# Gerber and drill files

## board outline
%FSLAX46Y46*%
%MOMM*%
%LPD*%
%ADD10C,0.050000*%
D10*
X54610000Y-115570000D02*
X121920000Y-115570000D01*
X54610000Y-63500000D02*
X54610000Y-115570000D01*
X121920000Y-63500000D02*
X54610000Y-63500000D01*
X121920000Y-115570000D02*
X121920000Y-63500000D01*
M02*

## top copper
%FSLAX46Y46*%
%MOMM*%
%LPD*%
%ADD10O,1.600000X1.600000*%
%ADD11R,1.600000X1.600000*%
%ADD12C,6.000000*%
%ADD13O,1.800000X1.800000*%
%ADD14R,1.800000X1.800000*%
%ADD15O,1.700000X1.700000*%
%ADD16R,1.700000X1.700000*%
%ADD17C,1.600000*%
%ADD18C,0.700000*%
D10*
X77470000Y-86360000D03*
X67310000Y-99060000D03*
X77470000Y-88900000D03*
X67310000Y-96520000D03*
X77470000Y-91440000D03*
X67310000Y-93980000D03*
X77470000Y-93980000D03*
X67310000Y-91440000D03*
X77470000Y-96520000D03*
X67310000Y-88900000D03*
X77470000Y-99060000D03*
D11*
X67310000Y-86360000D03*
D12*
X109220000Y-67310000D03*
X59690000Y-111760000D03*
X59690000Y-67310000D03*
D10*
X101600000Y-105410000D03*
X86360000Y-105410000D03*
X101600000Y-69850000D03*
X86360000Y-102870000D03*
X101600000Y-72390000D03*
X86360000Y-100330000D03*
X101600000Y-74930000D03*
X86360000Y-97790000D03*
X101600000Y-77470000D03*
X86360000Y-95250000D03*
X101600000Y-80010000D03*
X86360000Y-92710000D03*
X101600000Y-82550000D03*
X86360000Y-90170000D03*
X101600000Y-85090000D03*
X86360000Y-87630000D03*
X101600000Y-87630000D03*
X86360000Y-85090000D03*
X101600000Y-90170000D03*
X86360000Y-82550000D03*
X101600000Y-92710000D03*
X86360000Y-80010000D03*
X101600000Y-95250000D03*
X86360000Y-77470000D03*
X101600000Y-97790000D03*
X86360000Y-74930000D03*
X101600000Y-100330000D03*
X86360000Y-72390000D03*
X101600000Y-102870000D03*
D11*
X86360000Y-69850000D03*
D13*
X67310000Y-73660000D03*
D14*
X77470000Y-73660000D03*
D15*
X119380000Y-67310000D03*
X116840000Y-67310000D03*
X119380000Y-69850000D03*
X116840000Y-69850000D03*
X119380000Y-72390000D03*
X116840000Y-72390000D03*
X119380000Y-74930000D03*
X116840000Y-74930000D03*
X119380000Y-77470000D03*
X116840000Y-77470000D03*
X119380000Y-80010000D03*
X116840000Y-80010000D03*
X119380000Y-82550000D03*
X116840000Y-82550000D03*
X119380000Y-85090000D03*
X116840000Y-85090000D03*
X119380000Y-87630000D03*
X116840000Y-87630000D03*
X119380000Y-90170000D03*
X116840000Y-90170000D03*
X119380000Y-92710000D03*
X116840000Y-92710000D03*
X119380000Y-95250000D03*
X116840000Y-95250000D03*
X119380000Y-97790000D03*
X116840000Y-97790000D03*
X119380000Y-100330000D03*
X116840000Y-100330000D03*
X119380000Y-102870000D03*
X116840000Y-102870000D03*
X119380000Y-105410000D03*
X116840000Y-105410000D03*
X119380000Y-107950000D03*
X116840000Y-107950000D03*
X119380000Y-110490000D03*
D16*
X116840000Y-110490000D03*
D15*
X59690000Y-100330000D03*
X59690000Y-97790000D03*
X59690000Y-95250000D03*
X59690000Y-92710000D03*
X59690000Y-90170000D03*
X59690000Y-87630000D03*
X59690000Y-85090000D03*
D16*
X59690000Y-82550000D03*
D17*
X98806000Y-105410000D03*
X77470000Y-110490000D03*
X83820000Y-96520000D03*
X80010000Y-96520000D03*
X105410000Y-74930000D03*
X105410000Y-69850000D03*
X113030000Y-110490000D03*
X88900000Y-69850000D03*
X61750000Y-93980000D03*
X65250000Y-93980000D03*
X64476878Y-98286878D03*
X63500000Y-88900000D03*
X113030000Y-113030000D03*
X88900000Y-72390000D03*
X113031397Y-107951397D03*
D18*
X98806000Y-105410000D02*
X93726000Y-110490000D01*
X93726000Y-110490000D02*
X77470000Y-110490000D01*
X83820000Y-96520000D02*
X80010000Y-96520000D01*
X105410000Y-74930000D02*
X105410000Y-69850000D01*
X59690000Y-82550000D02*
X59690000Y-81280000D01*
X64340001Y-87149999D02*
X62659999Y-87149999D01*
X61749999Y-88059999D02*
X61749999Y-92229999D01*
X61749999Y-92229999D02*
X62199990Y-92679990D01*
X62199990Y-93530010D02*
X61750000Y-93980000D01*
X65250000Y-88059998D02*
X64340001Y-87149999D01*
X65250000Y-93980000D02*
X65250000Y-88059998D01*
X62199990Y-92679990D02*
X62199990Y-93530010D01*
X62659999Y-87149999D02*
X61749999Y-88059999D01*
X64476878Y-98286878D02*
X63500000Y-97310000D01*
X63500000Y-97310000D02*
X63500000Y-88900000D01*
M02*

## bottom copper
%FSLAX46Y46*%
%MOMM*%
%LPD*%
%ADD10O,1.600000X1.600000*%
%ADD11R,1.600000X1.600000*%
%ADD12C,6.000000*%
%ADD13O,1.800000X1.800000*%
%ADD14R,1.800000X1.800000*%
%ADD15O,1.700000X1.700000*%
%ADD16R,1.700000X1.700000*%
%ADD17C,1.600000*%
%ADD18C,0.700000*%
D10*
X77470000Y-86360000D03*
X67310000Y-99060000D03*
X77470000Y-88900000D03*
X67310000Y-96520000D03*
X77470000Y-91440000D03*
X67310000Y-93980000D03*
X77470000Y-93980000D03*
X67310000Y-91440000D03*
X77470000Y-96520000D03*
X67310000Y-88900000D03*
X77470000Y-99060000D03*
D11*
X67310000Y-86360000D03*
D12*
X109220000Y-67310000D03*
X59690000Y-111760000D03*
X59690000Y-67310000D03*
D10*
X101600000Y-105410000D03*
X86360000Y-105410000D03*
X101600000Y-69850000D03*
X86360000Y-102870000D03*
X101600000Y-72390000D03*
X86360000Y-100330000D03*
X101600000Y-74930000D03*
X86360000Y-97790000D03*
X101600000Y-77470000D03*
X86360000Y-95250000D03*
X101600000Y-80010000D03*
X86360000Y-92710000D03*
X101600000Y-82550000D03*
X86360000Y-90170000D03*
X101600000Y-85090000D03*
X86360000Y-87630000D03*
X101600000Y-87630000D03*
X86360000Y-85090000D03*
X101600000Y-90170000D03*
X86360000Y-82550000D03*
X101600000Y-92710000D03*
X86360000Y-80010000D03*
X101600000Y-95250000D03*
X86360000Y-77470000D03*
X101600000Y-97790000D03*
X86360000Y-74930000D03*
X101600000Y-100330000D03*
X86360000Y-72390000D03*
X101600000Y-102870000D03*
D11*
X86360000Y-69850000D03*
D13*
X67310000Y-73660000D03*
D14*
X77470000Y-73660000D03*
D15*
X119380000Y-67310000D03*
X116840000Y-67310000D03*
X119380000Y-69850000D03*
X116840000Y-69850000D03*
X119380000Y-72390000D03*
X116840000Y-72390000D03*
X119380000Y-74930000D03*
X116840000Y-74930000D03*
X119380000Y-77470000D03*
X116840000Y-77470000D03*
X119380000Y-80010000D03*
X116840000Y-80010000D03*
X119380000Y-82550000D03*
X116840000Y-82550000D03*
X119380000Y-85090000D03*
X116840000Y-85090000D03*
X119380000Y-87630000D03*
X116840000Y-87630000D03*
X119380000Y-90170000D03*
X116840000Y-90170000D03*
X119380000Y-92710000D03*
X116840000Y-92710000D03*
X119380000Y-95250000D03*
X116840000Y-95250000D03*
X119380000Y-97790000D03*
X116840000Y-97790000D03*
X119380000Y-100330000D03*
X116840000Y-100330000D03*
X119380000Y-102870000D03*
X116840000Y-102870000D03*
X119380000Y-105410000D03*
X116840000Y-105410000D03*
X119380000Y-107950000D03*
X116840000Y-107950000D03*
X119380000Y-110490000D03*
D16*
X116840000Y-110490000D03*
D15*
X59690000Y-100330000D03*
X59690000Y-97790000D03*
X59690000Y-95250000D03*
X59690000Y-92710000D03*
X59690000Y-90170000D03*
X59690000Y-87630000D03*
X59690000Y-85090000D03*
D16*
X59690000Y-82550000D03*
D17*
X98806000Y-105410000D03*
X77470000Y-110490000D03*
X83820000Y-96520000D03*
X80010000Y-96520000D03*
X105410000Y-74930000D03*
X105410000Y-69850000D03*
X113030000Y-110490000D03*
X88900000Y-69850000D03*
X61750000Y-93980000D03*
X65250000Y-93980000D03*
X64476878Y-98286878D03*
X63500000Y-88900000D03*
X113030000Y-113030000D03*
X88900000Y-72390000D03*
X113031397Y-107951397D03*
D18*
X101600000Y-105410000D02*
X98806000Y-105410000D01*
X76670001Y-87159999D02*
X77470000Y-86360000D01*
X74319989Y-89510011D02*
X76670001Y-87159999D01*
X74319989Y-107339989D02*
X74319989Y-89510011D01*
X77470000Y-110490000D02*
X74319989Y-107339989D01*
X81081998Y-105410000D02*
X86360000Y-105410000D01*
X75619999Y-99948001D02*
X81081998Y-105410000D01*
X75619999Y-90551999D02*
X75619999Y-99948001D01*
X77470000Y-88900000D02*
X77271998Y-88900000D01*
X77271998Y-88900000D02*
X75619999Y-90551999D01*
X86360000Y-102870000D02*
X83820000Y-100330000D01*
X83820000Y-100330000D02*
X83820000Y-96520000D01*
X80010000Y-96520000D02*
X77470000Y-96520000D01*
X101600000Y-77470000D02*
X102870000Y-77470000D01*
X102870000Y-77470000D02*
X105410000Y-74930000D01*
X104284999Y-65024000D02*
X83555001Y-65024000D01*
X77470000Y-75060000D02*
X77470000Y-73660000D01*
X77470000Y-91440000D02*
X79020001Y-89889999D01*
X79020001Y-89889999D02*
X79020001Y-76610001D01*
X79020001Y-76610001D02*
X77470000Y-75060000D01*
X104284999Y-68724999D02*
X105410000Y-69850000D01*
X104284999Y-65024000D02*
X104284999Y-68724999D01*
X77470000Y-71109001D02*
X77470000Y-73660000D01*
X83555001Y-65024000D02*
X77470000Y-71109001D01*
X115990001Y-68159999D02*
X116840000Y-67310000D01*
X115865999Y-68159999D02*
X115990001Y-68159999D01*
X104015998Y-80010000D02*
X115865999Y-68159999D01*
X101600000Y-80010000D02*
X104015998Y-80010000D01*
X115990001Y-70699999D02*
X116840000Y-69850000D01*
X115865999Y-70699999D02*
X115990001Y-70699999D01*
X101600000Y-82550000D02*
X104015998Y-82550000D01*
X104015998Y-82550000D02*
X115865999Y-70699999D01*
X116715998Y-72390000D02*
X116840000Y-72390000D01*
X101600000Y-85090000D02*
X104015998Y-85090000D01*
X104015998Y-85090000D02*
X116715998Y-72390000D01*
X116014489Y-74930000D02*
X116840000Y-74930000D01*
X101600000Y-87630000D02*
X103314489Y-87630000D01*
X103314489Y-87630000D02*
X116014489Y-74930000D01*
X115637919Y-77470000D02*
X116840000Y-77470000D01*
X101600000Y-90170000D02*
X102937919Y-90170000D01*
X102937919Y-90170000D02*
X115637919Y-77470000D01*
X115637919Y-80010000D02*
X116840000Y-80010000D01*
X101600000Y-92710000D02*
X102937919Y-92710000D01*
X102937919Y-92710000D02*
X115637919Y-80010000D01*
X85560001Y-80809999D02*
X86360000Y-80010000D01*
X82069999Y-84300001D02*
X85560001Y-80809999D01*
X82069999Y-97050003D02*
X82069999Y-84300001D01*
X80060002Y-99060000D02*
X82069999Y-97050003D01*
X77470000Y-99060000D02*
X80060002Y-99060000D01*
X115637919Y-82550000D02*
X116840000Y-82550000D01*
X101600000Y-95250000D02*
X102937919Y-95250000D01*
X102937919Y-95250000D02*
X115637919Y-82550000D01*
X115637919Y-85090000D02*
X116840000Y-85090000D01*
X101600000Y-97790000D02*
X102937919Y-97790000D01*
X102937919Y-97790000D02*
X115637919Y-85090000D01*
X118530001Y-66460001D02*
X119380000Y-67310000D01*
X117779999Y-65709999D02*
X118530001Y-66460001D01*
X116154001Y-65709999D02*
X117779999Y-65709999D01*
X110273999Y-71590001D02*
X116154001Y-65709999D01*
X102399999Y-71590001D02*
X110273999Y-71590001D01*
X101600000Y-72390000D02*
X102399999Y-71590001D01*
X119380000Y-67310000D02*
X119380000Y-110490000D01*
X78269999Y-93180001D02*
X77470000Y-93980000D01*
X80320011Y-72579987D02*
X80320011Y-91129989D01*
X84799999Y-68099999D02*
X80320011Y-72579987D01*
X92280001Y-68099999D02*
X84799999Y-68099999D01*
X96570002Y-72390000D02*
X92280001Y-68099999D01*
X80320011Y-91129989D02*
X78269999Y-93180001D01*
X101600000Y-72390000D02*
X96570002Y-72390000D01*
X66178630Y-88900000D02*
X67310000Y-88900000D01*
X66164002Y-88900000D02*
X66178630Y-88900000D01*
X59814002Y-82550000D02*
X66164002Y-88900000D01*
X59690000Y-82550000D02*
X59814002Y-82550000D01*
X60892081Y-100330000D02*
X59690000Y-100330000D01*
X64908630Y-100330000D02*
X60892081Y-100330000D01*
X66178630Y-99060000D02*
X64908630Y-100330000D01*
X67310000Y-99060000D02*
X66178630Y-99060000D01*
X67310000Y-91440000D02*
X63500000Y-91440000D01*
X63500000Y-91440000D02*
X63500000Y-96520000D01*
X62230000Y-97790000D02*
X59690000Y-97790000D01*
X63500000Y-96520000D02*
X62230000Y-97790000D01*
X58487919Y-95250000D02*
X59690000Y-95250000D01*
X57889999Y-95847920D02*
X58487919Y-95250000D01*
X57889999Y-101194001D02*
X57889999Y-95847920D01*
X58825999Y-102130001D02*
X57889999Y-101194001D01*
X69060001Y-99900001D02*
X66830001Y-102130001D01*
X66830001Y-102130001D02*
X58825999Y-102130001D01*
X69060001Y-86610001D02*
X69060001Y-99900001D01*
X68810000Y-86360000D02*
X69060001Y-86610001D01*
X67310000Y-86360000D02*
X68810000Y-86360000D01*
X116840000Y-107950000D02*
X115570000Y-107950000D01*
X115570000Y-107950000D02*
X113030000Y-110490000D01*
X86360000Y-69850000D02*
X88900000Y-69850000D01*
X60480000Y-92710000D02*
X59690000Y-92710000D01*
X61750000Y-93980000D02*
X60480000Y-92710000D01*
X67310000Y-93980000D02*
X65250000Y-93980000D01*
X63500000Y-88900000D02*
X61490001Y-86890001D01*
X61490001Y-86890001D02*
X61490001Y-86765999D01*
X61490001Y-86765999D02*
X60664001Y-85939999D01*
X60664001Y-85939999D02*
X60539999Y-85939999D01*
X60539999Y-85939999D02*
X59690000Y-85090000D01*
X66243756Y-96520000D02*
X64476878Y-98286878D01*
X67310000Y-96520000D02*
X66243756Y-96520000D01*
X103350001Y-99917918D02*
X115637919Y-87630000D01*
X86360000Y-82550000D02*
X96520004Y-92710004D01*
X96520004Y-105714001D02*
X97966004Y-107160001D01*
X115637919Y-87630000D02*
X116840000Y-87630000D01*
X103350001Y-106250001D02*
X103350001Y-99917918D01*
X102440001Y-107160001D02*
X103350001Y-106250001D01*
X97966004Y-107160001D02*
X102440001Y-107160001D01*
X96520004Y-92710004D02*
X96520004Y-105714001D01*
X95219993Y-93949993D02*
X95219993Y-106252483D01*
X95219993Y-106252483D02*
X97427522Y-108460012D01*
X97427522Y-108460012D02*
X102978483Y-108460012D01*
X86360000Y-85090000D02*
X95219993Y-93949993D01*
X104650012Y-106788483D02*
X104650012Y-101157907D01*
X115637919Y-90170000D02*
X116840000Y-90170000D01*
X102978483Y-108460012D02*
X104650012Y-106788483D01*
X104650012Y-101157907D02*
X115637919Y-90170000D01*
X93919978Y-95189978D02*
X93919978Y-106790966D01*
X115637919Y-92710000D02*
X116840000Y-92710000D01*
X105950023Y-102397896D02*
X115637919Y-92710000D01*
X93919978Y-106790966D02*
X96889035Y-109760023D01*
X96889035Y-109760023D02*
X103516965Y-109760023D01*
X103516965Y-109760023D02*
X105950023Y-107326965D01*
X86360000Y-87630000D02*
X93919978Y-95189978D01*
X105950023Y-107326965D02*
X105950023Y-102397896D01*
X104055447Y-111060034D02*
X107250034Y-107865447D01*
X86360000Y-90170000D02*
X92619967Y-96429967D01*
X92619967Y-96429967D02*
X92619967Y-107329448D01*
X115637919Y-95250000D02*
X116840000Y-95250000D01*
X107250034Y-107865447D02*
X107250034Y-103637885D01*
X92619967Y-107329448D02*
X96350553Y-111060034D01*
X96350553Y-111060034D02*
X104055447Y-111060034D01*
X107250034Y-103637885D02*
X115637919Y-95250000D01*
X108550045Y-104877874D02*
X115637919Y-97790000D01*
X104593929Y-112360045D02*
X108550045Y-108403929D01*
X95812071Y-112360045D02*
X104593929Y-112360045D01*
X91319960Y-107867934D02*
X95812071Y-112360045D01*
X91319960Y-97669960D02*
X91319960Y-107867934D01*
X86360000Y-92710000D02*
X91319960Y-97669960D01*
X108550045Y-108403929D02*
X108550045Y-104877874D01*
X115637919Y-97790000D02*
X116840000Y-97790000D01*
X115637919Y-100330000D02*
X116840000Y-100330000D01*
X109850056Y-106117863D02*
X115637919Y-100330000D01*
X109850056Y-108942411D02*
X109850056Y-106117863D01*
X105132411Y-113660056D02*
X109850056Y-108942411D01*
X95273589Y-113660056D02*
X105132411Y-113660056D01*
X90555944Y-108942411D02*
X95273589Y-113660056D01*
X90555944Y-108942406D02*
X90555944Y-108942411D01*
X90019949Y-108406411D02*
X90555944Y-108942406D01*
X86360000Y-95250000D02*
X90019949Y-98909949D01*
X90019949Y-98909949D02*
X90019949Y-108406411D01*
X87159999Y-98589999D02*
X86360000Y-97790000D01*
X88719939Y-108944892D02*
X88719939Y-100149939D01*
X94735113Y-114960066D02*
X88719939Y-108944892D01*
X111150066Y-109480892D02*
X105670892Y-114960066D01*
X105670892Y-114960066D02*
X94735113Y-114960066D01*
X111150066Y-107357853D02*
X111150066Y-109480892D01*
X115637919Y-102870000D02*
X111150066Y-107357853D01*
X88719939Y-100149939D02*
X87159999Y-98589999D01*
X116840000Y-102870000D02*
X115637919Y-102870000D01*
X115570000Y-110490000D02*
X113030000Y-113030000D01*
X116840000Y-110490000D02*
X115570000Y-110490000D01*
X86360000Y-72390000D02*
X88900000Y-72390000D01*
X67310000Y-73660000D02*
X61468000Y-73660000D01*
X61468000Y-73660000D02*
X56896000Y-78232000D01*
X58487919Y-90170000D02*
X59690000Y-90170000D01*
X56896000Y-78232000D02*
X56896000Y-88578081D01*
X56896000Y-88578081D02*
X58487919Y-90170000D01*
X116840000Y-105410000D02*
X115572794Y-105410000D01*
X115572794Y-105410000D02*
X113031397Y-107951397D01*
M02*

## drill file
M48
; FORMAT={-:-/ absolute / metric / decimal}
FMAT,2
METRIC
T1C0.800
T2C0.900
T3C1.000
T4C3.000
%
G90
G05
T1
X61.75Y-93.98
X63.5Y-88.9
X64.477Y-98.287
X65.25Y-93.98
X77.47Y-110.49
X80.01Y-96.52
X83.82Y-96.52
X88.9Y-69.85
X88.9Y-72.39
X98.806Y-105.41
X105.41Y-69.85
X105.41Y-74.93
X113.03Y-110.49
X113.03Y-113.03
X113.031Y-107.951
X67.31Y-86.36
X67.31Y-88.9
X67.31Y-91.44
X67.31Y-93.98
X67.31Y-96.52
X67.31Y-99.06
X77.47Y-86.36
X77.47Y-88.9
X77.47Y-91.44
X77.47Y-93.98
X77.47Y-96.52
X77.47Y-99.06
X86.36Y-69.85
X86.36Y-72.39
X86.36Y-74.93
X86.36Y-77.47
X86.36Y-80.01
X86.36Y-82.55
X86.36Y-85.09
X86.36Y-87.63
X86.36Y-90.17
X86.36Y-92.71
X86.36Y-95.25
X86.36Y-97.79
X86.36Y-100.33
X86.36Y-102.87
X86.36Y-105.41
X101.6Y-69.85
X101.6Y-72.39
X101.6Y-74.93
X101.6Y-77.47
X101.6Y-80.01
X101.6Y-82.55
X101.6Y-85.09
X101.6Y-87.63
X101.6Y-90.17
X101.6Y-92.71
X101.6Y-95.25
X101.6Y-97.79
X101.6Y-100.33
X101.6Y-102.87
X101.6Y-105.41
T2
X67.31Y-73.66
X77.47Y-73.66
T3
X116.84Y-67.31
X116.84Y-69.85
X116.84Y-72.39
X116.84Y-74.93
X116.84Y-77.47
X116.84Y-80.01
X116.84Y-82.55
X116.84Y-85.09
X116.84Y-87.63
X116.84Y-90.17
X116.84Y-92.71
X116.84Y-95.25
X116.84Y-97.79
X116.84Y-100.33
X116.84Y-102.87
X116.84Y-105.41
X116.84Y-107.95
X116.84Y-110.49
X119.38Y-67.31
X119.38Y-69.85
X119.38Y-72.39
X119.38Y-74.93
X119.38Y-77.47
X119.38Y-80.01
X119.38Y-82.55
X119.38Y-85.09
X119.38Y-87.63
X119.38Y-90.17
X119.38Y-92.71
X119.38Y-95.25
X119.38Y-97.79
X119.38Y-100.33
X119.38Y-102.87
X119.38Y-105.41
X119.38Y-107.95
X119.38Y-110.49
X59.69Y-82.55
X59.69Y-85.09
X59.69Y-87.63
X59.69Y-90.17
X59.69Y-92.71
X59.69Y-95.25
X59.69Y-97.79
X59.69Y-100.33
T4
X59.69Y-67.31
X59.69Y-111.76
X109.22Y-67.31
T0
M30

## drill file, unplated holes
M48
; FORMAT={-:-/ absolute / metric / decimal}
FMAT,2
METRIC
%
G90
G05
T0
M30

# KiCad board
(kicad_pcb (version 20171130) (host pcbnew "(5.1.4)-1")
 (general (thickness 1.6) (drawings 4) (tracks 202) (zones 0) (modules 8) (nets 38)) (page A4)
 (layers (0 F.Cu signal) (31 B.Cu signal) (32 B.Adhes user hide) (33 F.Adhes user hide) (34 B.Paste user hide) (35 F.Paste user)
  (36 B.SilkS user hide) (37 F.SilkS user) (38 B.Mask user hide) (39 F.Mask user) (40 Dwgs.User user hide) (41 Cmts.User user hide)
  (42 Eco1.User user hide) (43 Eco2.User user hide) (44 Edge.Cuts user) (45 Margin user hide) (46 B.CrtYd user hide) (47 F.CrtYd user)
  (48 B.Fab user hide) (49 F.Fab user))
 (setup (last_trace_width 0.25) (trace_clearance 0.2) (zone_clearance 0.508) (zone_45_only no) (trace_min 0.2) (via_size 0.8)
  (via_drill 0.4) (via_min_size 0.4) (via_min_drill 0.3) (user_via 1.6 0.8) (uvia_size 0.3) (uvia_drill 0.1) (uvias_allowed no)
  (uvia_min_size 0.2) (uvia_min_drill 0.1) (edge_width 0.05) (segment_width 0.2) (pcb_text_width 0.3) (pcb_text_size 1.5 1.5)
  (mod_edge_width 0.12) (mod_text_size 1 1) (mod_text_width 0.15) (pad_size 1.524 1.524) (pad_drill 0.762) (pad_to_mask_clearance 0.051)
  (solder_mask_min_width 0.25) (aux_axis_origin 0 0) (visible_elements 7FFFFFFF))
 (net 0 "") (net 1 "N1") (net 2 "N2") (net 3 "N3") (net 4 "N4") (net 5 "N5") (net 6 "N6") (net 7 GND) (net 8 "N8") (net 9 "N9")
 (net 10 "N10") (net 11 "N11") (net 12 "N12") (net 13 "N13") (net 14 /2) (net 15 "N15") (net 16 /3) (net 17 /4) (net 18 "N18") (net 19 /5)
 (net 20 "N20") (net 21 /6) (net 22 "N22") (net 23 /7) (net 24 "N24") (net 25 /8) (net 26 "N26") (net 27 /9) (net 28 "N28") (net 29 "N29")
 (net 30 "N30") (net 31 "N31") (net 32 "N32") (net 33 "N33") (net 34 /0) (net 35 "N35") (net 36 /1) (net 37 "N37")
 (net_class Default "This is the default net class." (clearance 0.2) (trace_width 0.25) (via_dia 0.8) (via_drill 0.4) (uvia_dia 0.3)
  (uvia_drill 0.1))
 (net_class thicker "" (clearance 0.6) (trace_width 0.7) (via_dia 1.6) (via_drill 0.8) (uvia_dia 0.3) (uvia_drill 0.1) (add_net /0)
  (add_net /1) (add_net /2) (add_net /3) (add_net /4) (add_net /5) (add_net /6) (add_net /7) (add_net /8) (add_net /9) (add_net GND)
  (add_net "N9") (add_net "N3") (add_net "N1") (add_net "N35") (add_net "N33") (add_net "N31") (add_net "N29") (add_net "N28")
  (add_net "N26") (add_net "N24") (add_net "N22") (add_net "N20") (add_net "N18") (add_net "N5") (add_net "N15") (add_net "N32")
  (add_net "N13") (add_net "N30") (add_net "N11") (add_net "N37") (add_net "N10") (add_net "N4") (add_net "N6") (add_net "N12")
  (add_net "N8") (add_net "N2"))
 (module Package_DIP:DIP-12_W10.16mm (layer F.Cu) (at 67.31 86.36)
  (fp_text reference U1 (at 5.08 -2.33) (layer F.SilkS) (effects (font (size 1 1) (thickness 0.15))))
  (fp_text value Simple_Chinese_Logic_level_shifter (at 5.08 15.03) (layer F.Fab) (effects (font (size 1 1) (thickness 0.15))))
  (pad 10 thru_hole oval (at 10.16 0) (size 1.6 1.6) (drill 0.8) (layers *.Cu *.Mask) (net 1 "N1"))
  (pad 5 thru_hole oval (at 0 12.7) (size 1.6 1.6) (drill 0.8) (layers *.Cu *.Mask) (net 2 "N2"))
  (pad 9 thru_hole oval (at 10.16 2.54) (size 1.6 1.6) (drill 0.8) (layers *.Cu *.Mask) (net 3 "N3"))
  (pad 4 thru_hole oval (at 0 10.16) (size 1.6 1.6) (drill 0.8) (layers *.Cu *.Mask) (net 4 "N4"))
  (pad 11 thru_hole oval (at 10.16 5.08) (size 1.6 1.6) (drill 0.8) (layers *.Cu *.Mask) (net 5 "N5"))
  (pad 12 thru_hole oval (at 0 7.62) (size 1.6 1.6) (drill 0.8) (layers *.Cu *.Mask) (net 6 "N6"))
  (pad 6 thru_hole oval (at 10.16 7.62) (size 1.6 1.6) (drill 0.8) (layers *.Cu *.Mask) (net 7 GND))
  (pad 1 thru_hole oval (at 0 5.08) (size 1.6 1.6) (drill 0.8) (layers *.Cu *.Mask) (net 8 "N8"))
  (pad 8 thru_hole oval (at 10.16 10.16) (size 1.6 1.6) (drill 0.8) (layers *.Cu *.Mask) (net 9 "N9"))
  (pad 3 thru_hole oval (at 0 2.54) (size 1.6 1.6) (drill 0.8) (layers *.Cu *.Mask) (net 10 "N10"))
  (pad 7 thru_hole oval (at 10.16 12.7) (size 1.6 1.6) (drill 0.8) (layers *.Cu *.Mask) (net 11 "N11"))
  (pad 2 thru_hole rect (at 0 0) (size 1.6 1.6) (drill 0.8) (layers *.Cu *.Mask) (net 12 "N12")))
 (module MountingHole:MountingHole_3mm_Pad (layer F.Cu) (at 109.22 67.31)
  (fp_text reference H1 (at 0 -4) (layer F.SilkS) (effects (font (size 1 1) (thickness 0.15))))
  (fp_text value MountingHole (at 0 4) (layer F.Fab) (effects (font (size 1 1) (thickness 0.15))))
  (pad 1 thru_hole circle (at 0 0) (size 6 6) (drill 3) (layers *.Cu *.Mask)))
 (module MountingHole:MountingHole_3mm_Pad (layer F.Cu) (at 59.69 111.76)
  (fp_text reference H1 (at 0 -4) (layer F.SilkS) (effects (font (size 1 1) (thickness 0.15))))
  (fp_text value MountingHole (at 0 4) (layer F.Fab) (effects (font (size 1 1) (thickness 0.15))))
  (pad 1 thru_hole circle (at 0 0) (size 6 6) (drill 3) (layers *.Cu *.Mask)))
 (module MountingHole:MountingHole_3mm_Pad (layer F.Cu) (at 59.69 67.31)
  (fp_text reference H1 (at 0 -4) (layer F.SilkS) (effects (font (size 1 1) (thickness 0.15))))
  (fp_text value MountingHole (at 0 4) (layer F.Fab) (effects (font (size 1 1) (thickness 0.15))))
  (pad 1 thru_hole circle (at 0 0) (size 6 6) (drill 3) (layers *.Cu *.Mask)))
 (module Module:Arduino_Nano (layer F.Cu) (at 86.36 69.85)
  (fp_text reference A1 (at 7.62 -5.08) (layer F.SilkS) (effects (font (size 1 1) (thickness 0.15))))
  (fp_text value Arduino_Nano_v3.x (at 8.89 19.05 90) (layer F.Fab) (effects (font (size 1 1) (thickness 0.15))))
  (pad 16 thru_hole oval (at 15.24 35.56) (size 1.6 1.6) (drill 0.8) (layers *.Cu *.Mask) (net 1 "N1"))
  (pad 15 thru_hole oval (at 0 35.56) (size 1.6 1.6) (drill 0.8) (layers *.Cu *.Mask) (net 3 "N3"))
  (pad 30 thru_hole oval (at 15.24 0) (size 1.6 1.6) (drill 0.8) (layers *.Cu *.Mask) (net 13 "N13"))
  (pad 14 thru_hole oval (at 0 33.02) (size 1.6 1.6) (drill 0.8) (layers *.Cu *.Mask) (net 9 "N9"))
  (pad 29 thru_hole oval (at 15.24 2.54) (size 1.6 1.6) (drill 0.8) (layers *.Cu *.Mask) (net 7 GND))
  (pad 13 thru_hole oval (at 0 30.48) (size 1.6 1.6) (drill 0.8) (layers *.Cu *.Mask) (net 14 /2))
  (pad 28 thru_hole oval (at 15.24 5.08) (size 1.6 1.6) (drill 0.8) (layers *.Cu *.Mask) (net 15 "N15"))
  (pad 12 thru_hole oval (at 0 27.94) (size 1.6 1.6) (drill 0.8) (layers *.Cu *.Mask) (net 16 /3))
  (pad 27 thru_hole oval (at 15.24 7.62) (size 1.6 1.6) (drill 0.8) (layers *.Cu *.Mask) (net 5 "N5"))
  (pad 11 thru_hole oval (at 0 25.4) (size 1.6 1.6) (drill 0.8) (layers *.Cu *.Mask) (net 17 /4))
  (pad 26 thru_hole oval (at 15.24 10.16) (size 1.6 1.6) (drill 0.8) (layers *.Cu *.Mask) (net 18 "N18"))
  (pad 10 thru_hole oval (at 0 22.86) (size 1.6 1.6) (drill 0.8) (layers *.Cu *.Mask) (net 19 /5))
  (pad 25 thru_hole oval (at 15.24 12.7) (size 1.6 1.6) (drill 0.8) (layers *.Cu *.Mask) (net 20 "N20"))
  (pad 9 thru_hole oval (at 0 20.32) (size 1.6 1.6) (drill 0.8) (layers *.Cu *.Mask) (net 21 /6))
  (pad 24 thru_hole oval (at 15.24 15.24) (size 1.6 1.6) (drill 0.8) (layers *.Cu *.Mask) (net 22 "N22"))
  (pad 8 thru_hole oval (at 0 17.78) (size 1.6 1.6) (drill 0.8) (layers *.Cu *.Mask) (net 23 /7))
  (pad 23 thru_hole oval (at 15.24 17.78) (size 1.6 1.6) (drill 0.8) (layers *.Cu *.Mask) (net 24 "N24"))
  (pad 7 thru_hole oval (at 0 15.24) (size 1.6 1.6) (drill 0.8) (layers *.Cu *.Mask) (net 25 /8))
  (pad 22 thru_hole oval (at 15.24 20.32) (size 1.6 1.6) (drill 0.8) (layers *.Cu *.Mask) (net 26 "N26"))
  (pad 6 thru_hole oval (at 0 12.7) (size 1.6 1.6) (drill 0.8) (layers *.Cu *.Mask) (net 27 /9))
  (pad 21 thru_hole oval (at 15.24 22.86) (size 1.6 1.6) (drill 0.8) (layers *.Cu *.Mask) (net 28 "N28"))
  (pad 5 thru_hole oval (at 0 10.16) (size 1.6 1.6) (drill 0.8) (layers *.Cu *.Mask) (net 11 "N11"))
  (pad 20 thru_hole oval (at 15.24 25.4) (size 1.6 1.6) (drill 0.8) (layers *.Cu *.Mask) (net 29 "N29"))
  (pad 4 thru_hole oval (at 0 7.62) (size 1.6 1.6) (drill 0.8) (layers *.Cu *.Mask) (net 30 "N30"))
  (pad 19 thru_hole oval (at 15.24 27.94) (size 1.6 1.6) (drill 0.8) (layers *.Cu *.Mask) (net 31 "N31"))
  (pad 3 thru_hole oval (at 0 5.08) (size 1.6 1.6) (drill 0.8) (layers *.Cu *.Mask) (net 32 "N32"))
  (pad 18 thru_hole oval (at 15.24 30.48) (size 1.6 1.6) (drill 0.8) (layers *.Cu *.Mask) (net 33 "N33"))
  (pad 2 thru_hole oval (at 0 2.54) (size 1.6 1.6) (drill 0.8) (layers *.Cu *.Mask) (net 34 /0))
  (pad 17 thru_hole oval (at 15.24 33.02) (size 1.6 1.6) (drill 0.8) (layers *.Cu *.Mask) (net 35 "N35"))
  (pad 1 thru_hole rect (at 0 0) (size 1.6 1.6) (drill 0.8) (layers *.Cu *.Mask) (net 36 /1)))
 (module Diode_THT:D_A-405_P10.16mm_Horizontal (layer F.Cu) (at 77.47 73.66 180)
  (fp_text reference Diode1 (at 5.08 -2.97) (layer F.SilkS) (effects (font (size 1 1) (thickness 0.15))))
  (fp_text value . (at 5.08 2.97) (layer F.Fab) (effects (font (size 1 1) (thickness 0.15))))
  (pad 2 thru_hole oval (at 10.16 0 180) (size 1.8 1.8) (drill 0.9) (layers *.Cu *.Mask) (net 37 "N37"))
  (pad 1 thru_hole rect (at 0 0 180) (size 1.8 1.8) (drill 0.9) (layers *.Cu *.Mask) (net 5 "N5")))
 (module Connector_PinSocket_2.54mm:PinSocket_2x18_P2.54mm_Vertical (layer F.Cu) (at 116.84 110.49 180)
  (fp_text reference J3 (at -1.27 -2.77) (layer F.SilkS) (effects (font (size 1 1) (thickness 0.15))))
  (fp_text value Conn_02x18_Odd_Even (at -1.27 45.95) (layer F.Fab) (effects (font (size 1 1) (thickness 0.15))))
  (pad 36 thru_hole oval (at -2.54 43.18 180) (size 1.7 1.7) (drill 1) (layers *.Cu *.Mask) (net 7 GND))
  (pad 35 thru_hole oval (at 0 43.18 180) (size 1.7 1.7) (drill 1) (layers *.Cu *.Mask) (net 18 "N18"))
  (pad 34 thru_hole oval (at -2.54 40.64 180) (size 1.7 1.7) (drill 1) (layers *.Cu *.Mask) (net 7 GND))
  (pad 33 thru_hole oval (at 0 40.64 180) (size 1.7 1.7) (drill 1) (layers *.Cu *.Mask) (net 20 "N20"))
  (pad 32 thru_hole oval (at -2.54 38.1 180) (size 1.7 1.7) (drill 1) (layers *.Cu *.Mask) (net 7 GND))
  (pad 31 thru_hole oval (at 0 38.1 180) (size 1.7 1.7) (drill 1) (layers *.Cu *.Mask) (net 22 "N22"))
  (pad 30 thru_hole oval (at -2.54 35.56 180) (size 1.7 1.7) (drill 1) (layers *.Cu *.Mask) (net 7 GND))
  (pad 29 thru_hole oval (at 0 35.56 180) (size 1.7 1.7) (drill 1) (layers *.Cu *.Mask) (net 24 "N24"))
  (pad 28 thru_hole oval (at -2.54 33.02 180) (size 1.7 1.7) (drill 1) (layers *.Cu *.Mask) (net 7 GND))
  (pad 27 thru_hole oval (at 0 33.02 180) (size 1.7 1.7) (drill 1) (layers *.Cu *.Mask) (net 26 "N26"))
  (pad 26 thru_hole oval (at -2.54 30.48 180) (size 1.7 1.7) (drill 1) (layers *.Cu *.Mask) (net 7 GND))
  (pad 25 thru_hole oval (at 0 30.48 180) (size 1.7 1.7) (drill 1) (layers *.Cu *.Mask) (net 28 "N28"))
  (pad 24 thru_hole oval (at -2.54 27.94 180) (size 1.7 1.7) (drill 1) (layers *.Cu *.Mask) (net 7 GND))
  (pad 23 thru_hole oval (at 0 27.94 180) (size 1.7 1.7) (drill 1) (layers *.Cu *.Mask) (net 29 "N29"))
  (pad 22 thru_hole oval (at -2.54 25.4 180) (size 1.7 1.7) (drill 1) (layers *.Cu *.Mask) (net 7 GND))
  (pad 21 thru_hole oval (at 0 25.4 180) (size 1.7 1.7) (drill 1) (layers *.Cu *.Mask) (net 31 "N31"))
  (pad 20 thru_hole oval (at -2.54 22.86 180) (size 1.7 1.7) (drill 1) (layers *.Cu *.Mask) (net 7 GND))
  (pad 19 thru_hole oval (at 0 22.86 180) (size 1.7 1.7) (drill 1) (layers *.Cu *.Mask) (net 27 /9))
  (pad 18 thru_hole oval (at -2.54 20.32 180) (size 1.7 1.7) (drill 1) (layers *.Cu *.Mask) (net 7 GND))
  (pad 17 thru_hole oval (at 0 20.32 180) (size 1.7 1.7) (drill 1) (layers *.Cu *.Mask) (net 25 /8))
  (pad 16 thru_hole oval (at -2.54 17.78 180) (size 1.7 1.7) (drill 1) (layers *.Cu *.Mask) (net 7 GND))
  (pad 15 thru_hole oval (at 0 17.78 180) (size 1.7 1.7) (drill 1) (layers *.Cu *.Mask) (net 23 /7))
  (pad 14 thru_hole oval (at -2.54 15.24 180) (size 1.7 1.7) (drill 1) (layers *.Cu *.Mask) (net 7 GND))
  (pad 13 thru_hole oval (at 0 15.24 180) (size 1.7 1.7) (drill 1) (layers *.Cu *.Mask) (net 21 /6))
  (pad 12 thru_hole oval (at -2.54 12.7 180) (size 1.7 1.7) (drill 1) (layers *.Cu *.Mask) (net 7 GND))
  (pad 11 thru_hole oval (at 0 12.7 180) (size 1.7 1.7) (drill 1) (layers *.Cu *.Mask) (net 19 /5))
  (pad 10 thru_hole oval (at -2.54 10.16 180) (size 1.7 1.7) (drill 1) (layers *.Cu *.Mask) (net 7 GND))
  (pad 9 thru_hole oval (at 0 10.16 180) (size 1.7 1.7) (drill 1) (layers *.Cu *.Mask) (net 17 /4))
  (pad 8 thru_hole oval (at -2.54 7.62 180) (size 1.7 1.7) (drill 1) (layers *.Cu *.Mask) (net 7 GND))
  (pad 7 thru_hole oval (at 0 7.62 180) (size 1.7 1.7) (drill 1) (layers *.Cu *.Mask) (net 16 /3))
  (pad 6 thru_hole oval (at -2.54 5.08 180) (size 1.7 1.7) (drill 1) (layers *.Cu *.Mask) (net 7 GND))
  (pad 5 thru_hole oval (at 0 5.08 180) (size 1.7 1.7) (drill 1) (layers *.Cu *.Mask) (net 14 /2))
  (pad 4 thru_hole oval (at -2.54 2.54 180) (size 1.7 1.7) (drill 1) (layers *.Cu *.Mask) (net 7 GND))
  (pad 3 thru_hole oval (at 0 2.54 180) (size 1.7 1.7) (drill 1) (layers *.Cu *.Mask) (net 36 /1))
  (pad 2 thru_hole oval (at -2.54 0 180) (size 1.7 1.7) (drill 1) (layers *.Cu *.Mask) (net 7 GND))
  (pad 1 thru_hole rect (at 0 0 180) (size 1.7 1.7) (drill 1) (layers *.Cu *.Mask) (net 34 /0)))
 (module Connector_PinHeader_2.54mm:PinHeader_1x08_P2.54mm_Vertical (layer F.Cu) (at 59.69 82.55)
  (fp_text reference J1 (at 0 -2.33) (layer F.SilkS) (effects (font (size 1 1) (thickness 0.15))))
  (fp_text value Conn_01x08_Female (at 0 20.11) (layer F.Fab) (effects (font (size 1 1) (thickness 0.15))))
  (pad 8 thru_hole oval (at 0 17.78) (size 1.7 1.7) (drill 1) (layers *.Cu *.Mask) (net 2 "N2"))
  (pad 7 thru_hole oval (at 0 15.24) (size 1.7 1.7) (drill 1) (layers *.Cu *.Mask) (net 8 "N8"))
  (pad 6 thru_hole oval (at 0 12.7) (size 1.7 1.7) (drill 1) (layers *.Cu *.Mask) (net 12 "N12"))
  (pad 5 thru_hole oval (at 0 10.16) (size 1.7 1.7) (drill 1) (layers *.Cu *.Mask) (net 6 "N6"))
  (pad 4 thru_hole oval (at 0 7.62) (size 1.7 1.7) (drill 1) (layers *.Cu *.Mask) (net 37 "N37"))
  (pad 3 thru_hole oval (at 0 5.08) (size 1.7 1.7) (drill 1) (layers *.Cu *.Mask) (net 6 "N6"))
  (pad 2 thru_hole oval (at 0 2.54) (size 1.7 1.7) (drill 1) (layers *.Cu *.Mask) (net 4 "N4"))
  (pad 1 thru_hole rect (at 0 0) (size 1.7 1.7) (drill 1) (layers *.Cu *.Mask) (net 10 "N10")))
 (gr_line (start 54.61 115.57) (end 121.92 115.57) (layer Edge.Cuts) (width 0.05))
 (gr_line (start 54.61 63.5) (end 54.61 115.57) (layer Edge.Cuts) (width 0.05))
 (gr_line (start 121.92 63.5) (end 54.61 63.5) (layer Edge.Cuts) (width 0.05))
 (gr_line (start 121.92 115.57) (end 121.92 63.5) (layer Edge.Cuts) (width 0.05))
 (via (at 98.806 105.41) (size 1.6) (drill 0.8) (layers F.Cu B.Cu) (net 1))
 (segment (start 101.6 105.41) (end 98.806 105.41) (width 0.7) (layer B.Cu) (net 1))
 (via (at 77.47 110.49) (size 1.6) (drill 0.8) (layers F.Cu B.Cu) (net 1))
 (segment (start 76.670001 87.159999) (end 77.47 86.36) (width 0.7) (layer B.Cu) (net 1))
 (segment (start 74.319989 89.510011) (end 76.670001 87.159999) (width 0.7) (layer B.Cu) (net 1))
 (segment (start 74.319989 107.339989) (end 74.319989 89.510011) (width 0.7) (layer B.Cu) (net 1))
 (segment (start 77.47 110.49) (end 74.319989 107.339989) (width 0.7) (layer B.Cu) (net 1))
 (segment (start 98.806 105.41) (end 93.726 110.49) (width 0.7) (layer F.Cu) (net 1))
 (segment (start 93.726 110.49) (end 77.47 110.49) (width 0.7) (layer F.Cu) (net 1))
 (segment (start 81.081998 105.41) (end 86.36 105.41) (width 0.7) (layer B.Cu) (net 3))
 (segment (start 75.619999 99.948001) (end 81.081998 105.41) (width 0.7) (layer B.Cu) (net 3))
 (segment (start 75.619999 90.551999) (end 75.619999 99.948001) (width 0.7) (layer B.Cu) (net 3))
 (segment (start 77.47 88.9) (end 77.271998 88.9) (width 0.7) (layer B.Cu) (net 3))
 (segment (start 77.271998 88.9) (end 75.619999 90.551999) (width 0.7) (layer B.Cu) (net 3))
 (segment (start 86.36 102.87) (end 83.82 100.33) (width 0.7) (layer B.Cu) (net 9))
 (via (at 83.82 96.52) (size 1.6) (drill 0.8) (layers F.Cu B.Cu) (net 9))
 (segment (start 83.82 100.33) (end 83.82 96.52) (width 0.7) (layer B.Cu) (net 9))
 (via (at 80.01 96.52) (size 1.6) (drill 0.8) (layers F.Cu B.Cu) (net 9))
 (segment (start 83.82 96.52) (end 80.01 96.52) (width 0.7) (layer F.Cu) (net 9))
 (segment (start 80.01 96.52) (end 77.47 96.52) (width 0.7) (layer B.Cu) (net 9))
 (via (at 105.41 74.93) (size 1.6) (drill 0.8) (layers F.Cu B.Cu) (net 5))
 (segment (start 101.6 77.47) (end 102.87 77.47) (width 0.7) (layer B.Cu) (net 5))
 (segment (start 102.87 77.47) (end 105.41 74.93) (width 0.7) (layer B.Cu) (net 5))
 (via (at 105.41 69.85) (size 1.6) (drill 0.8) (layers F.Cu B.Cu) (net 5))
 (segment (start 105.41 74.93) (end 105.41 69.85) (width 0.7) (layer F.Cu) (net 5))
 (segment (start 104.284999 65.024) (end 83.555001 65.024) (width 0.7) (layer B.Cu) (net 5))
 (segment (start 77.47 75.06) (end 77.47 73.66) (width 0.7) (layer B.Cu) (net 5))
 (segment (start 77.47 91.44) (end 79.020001 89.889999) (width 0.7) (layer B.Cu) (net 5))
 (segment (start 79.020001 89.889999) (end 79.020001 76.610001) (width 0.7) (layer B.Cu) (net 5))
 (segment (start 79.020001 76.610001) (end 77.47 75.06) (width 0.7) (layer B.Cu) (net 5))
 (segment (start 104.284999 68.724999) (end 105.41 69.85) (width 0.7) (layer B.Cu) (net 5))
 (segment (start 104.284999 65.024) (end 104.284999 68.724999) (width 0.7) (layer B.Cu) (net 5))
 (segment (start 77.47 71.109001) (end 77.47 73.66) (width 0.7) (layer B.Cu) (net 5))
 (segment (start 83.555001 65.024) (end 77.47 71.109001) (width 0.7) (layer B.Cu) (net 5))
 (segment (start 115.990001 68.159999) (end 116.84 67.31) (width 0.7) (layer B.Cu) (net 18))
 (segment (start 115.865999 68.159999) (end 115.990001 68.159999) (width 0.7) (layer B.Cu) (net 18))
 (segment (start 104.015998 80.01) (end 115.865999 68.159999) (width 0.7) (layer B.Cu) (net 18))
 (segment (start 101.6 80.01) (end 104.015998 80.01) (width 0.7) (layer B.Cu) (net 18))
 (segment (start 115.990001 70.699999) (end 116.84 69.85) (width 0.7) (layer B.Cu) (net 20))
 (segment (start 115.865999 70.699999) (end 115.990001 70.699999) (width 0.7) (layer B.Cu) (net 20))
 (segment (start 101.6 82.55) (end 104.015998 82.55) (width 0.7) (layer B.Cu) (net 20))
 (segment (start 104.015998 82.55) (end 115.865999 70.699999) (width 0.7) (layer B.Cu) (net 20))
 (segment (start 116.715998 72.39) (end 116.84 72.39) (width 0.7) (layer B.Cu) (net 22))
 (segment (start 101.6 85.09) (end 104.015998 85.09) (width 0.7) (layer B.Cu) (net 22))
 (segment (start 104.015998 85.09) (end 116.715998 72.39) (width 0.7) (layer B.Cu) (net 22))
 (segment (start 116.014489 74.93) (end 116.84 74.93) (width 0.7) (layer B.Cu) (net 24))
 (segment (start 101.6 87.63) (end 103.314489 87.63) (width 0.7) (layer B.Cu) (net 24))
 (segment (start 103.314489 87.63) (end 116.014489 74.93) (width 0.7) (layer B.Cu) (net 24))
 (segment (start 115.637919 77.47) (end 116.84 77.47) (width 0.7) (layer B.Cu) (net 26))
 (segment (start 101.6 90.17) (end 102.937919 90.17) (width 0.7) (layer B.Cu) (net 26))
 (segment (start 102.937919 90.17) (end 115.637919 77.47) (width 0.7) (layer B.Cu) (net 26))
 (segment (start 115.637919 80.01) (end 116.84 80.01) (width 0.7) (layer B.Cu) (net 28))
 (segment (start 101.6 92.71) (end 102.937919 92.71) (width 0.7) (layer B.Cu) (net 28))
 (segment (start 102.937919 92.71) (end 115.637919 80.01) (width 0.7) (layer B.Cu) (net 28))
 (segment (start 85.560001 80.809999) (end 86.36 80.01) (width 0.7) (layer B.Cu) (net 11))
 (segment (start 82.069999 84.300001) (end 85.560001 80.809999) (width 0.7) (layer B.Cu) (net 11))
 (segment (start 82.069999 97.050003) (end 82.069999 84.300001) (width 0.7) (layer B.Cu) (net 11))
 (segment (start 80.060002 99.06) (end 82.069999 97.050003) (width 0.7) (layer B.Cu) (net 11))
 (segment (start 77.47 99.06) (end 80.060002 99.06) (width 0.7) (layer B.Cu) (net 11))
 (segment (start 115.637919 82.55) (end 116.84 82.55) (width 0.7) (layer B.Cu) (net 29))
 (segment (start 101.6 95.25) (end 102.937919 95.25) (width 0.7) (layer B.Cu) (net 29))
 (segment (start 102.937919 95.25) (end 115.637919 82.55) (width 0.7) (layer B.Cu) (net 29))
 (segment (start 115.637919 85.09) (end 116.84 85.09) (width 0.7) (layer B.Cu) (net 31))
 (segment (start 101.6 97.79) (end 102.937919 97.79) (width 0.7) (layer B.Cu) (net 31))
 (segment (start 102.937919 97.79) (end 115.637919 85.09) (width 0.7) (layer B.Cu) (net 31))
 (segment (start 118.530001 66.460001) (end 119.38 67.31) (width 0.7) (layer B.Cu) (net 7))
 (segment (start 117.779999 65.709999) (end 118.530001 66.460001) (width 0.7) (layer B.Cu) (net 7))
 (segment (start 116.154001 65.709999) (end 117.779999 65.709999) (width 0.7) (layer B.Cu) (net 7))
 (segment (start 110.273999 71.590001) (end 116.154001 65.709999) (width 0.7) (layer B.Cu) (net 7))
 (segment (start 102.399999 71.590001) (end 110.273999 71.590001) (width 0.7) (layer B.Cu) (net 7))
 (segment (start 101.6 72.39) (end 102.399999 71.590001) (width 0.7) (layer B.Cu) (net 7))
 (segment (start 119.38 67.31) (end 119.38 110.49) (width 0.7) (layer B.Cu) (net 7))
 (segment (start 78.269999 93.180001) (end 77.47 93.98) (width 0.7) (layer B.Cu) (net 7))
 (segment (start 80.320011 72.579987) (end 80.320011 91.129989) (width 0.7) (layer B.Cu) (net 7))
 (segment (start 84.799999 68.099999) (end 80.320011 72.579987) (width 0.7) (layer B.Cu) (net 7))
 (segment (start 92.280001 68.099999) (end 84.799999 68.099999) (width 0.7) (layer B.Cu) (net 7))
 (segment (start 96.570002 72.39) (end 92.280001 68.099999) (width 0.7) (layer B.Cu) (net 7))
 (segment (start 80.320011 91.129989) (end 78.269999 93.180001) (width 0.7) (layer B.Cu) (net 7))
 (segment (start 101.6 72.39) (end 96.570002 72.39) (width 0.7) (layer B.Cu) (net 7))
 (segment (start 59.69 82.55) (end 59.69 81.28) (width 0.7) (layer F.Cu) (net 10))
 (segment (start 66.17863 88.9) (end 67.31 88.9) (width 0.7) (layer B.Cu) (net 10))
 (segment (start 66.164002 88.9) (end 66.17863 88.9) (width 0.7) (layer B.Cu) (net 10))
 (segment (start 59.814002 82.55) (end 66.164002 88.9) (width 0.7) (layer B.Cu) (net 10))
 (segment (start 59.69 82.55) (end 59.814002 82.55) (width 0.7) (layer B.Cu) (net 10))
 (segment (start 60.892081 100.33) (end 59.69 100.33) (width 0.7) (layer B.Cu) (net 2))
 (segment (start 64.90863 100.33) (end 60.892081 100.33) (width 0.7) (layer B.Cu) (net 2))
 (segment (start 66.17863 99.06) (end 64.90863 100.33) (width 0.7) (layer B.Cu) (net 2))
 (segment (start 67.31 99.06) (end 66.17863 99.06) (width 0.7) (layer B.Cu) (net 2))
 (segment (start 67.31 91.44) (end 63.5 91.44) (width 0.7) (layer B.Cu) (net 8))
 (segment (start 63.5 91.44) (end 63.5 96.52) (width 0.7) (layer B.Cu) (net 8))
 (segment (start 62.23 97.79) (end 59.69 97.79) (width 0.7) (layer B.Cu) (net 8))
 (segment (start 63.5 96.52) (end 62.23 97.79) (width 0.7) (layer B.Cu) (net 8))
 (segment (start 58.487919 95.25) (end 59.69 95.25) (width 0.7) (layer B.Cu) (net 12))
 (segment (start 57.889999 95.84792) (end 58.487919 95.25) (width 0.7) (layer B.Cu) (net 12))
 (segment (start 57.889999 101.194001) (end 57.889999 95.84792) (width 0.7) (layer B.Cu) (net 12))
 (segment (start 58.825999 102.130001) (end 57.889999 101.194001) (width 0.7) (layer B.Cu) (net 12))
 (segment (start 69.060001 99.900001) (end 66.830001 102.130001) (width 0.7) (layer B.Cu) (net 12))
 (segment (start 66.830001 102.130001) (end 58.825999 102.130001) (width 0.7) (layer B.Cu) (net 12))
 (segment (start 69.060001 86.610001) (end 69.060001 99.900001) (width 0.7) (layer B.Cu) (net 12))
 (segment (start 68.81 86.36) (end 69.060001 86.610001) (width 0.7) (layer B.Cu) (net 12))
 (segment (start 67.31 86.36) (end 68.81 86.36) (width 0.7) (layer B.Cu) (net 12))
 (via (at 113.03 110.49) (size 1.6) (drill 0.8) (layers F.Cu B.Cu) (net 36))
 (segment (start 116.84 107.95) (end 115.57 107.95) (width 0.7) (layer B.Cu) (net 36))
 (segment (start 115.57 107.95) (end 113.03 110.49) (width 0.7) (layer B.Cu) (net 36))
 (segment (start 86.36 69.85) (end 88.9 69.85) (width 0.7) (layer B.Cu) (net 36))
 (via (at 88.9 69.85) (size 1.6) (drill 0.8) (layers F.Cu B.Cu) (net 36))
 (via (at 61.75 93.98) (size 1.6) (drill 0.8) (layers F.Cu B.Cu) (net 6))
 (via (at 65.25 93.98) (size 1.6) (drill 0.8) (layers F.Cu B.Cu) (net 6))
 (segment (start 64.340001 87.149999) (end 62.659999 87.149999) (width 0.7) (layer F.Cu) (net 6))
 (segment (start 61.749999 88.059999) (end 61.749999 92.229999) (width 0.7) (layer F.Cu) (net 6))
 (segment (start 61.749999 92.229999) (end 62.19999 92.67999) (width 0.7) (layer F.Cu) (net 6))
 (segment (start 60.48 92.71) (end 59.69 92.71) (width 0.7) (layer B.Cu) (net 6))
 (segment (start 62.19999 93.53001) (end 61.75 93.98) (width 0.7) (layer F.Cu) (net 6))
 (segment (start 65.25 88.059998) (end 64.340001 87.149999) (width 0.7) (layer F.Cu) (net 6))
 (segment (start 65.25 93.98) (end 65.25 88.059998) (width 0.7) (layer F.Cu) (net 6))
 (segment (start 62.19999 92.67999) (end 62.19999 93.53001) (width 0.7) (layer F.Cu) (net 6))
 (segment (start 61.75 93.98) (end 60.48 92.71) (width 0.7) (layer B.Cu) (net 6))
 (segment (start 62.659999 87.149999) (end 61.749999 88.059999) (width 0.7) (layer F.Cu) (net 6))
 (segment (start 67.31 93.98) (end 65.25 93.98) (width 0.7) (layer B.Cu) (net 6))
 (via (at 64.476878 98.286878) (size 1.6) (drill 0.8) (layers F.Cu B.Cu) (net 4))
 (segment (start 63.5 88.9) (end 61.490001 86.890001) (width 0.7) (layer B.Cu) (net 4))
 (segment (start 61.490001 86.890001) (end 61.490001 86.765999) (width 0.7) (layer B.Cu) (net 4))
 (segment (start 61.490001 86.765999) (end 60.664001 85.939999) (width 0.7) (layer B.Cu) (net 4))
 (segment (start 60.664001 85.939999) (end 60.539999 85.939999) (width 0.7) (layer B.Cu) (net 4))
 (segment (start 60.539999 85.939999) (end 59.69 85.09) (width 0.7) (layer B.Cu) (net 4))
 (via (at 63.5 88.9) (size 1.6) (drill 0.8) (layers F.Cu B.Cu) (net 4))
 (segment (start 66.243756 96.52) (end 64.476878 98.286878) (width 0.7) (layer B.Cu) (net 4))
 (segment (start 67.31 96.52) (end 66.243756 96.52) (width 0.7) (layer B.Cu) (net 4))
 (segment (start 64.476878 98.286878) (end 63.5 97.31) (width 0.7) (layer F.Cu) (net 4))
 (segment (start 63.5 97.31) (end 63.5 88.9) (width 0.7) (layer F.Cu) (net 4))
 (segment (start 103.350001 99.917918) (end 115.637919 87.63) (width 0.7) (layer B.Cu) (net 27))
 (segment (start 86.36 82.55) (end 96.520004 92.710004) (width 0.7) (layer B.Cu) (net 27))
 (segment (start 96.520004 105.714001) (end 97.966004 107.160001) (width 0.7) (layer B.Cu) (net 27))
 (segment (start 115.637919 87.63) (end 116.84 87.63) (width 0.7) (layer B.Cu) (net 27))
 (segment (start 103.350001 106.250001) (end 103.350001 99.917918) (width 0.7) (layer B.Cu) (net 27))
 (segment (start 102.440001 107.160001) (end 103.350001 106.250001) (width 0.7) (layer B.Cu) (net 27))
 (segment (start 97.966004 107.160001) (end 102.440001 107.160001) (width 0.7) (layer B.Cu) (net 27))
 (segment (start 96.520004 92.710004) (end 96.520004 105.714001) (width 0.7) (layer B.Cu) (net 27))
 (segment (start 95.219993 93.949993) (end 95.219993 106.252483) (width 0.7) (layer B.Cu) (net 25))
 (segment (start 95.219993 106.252483) (end 97.427522 108.460012) (width 0.7) (layer B.Cu) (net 25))
 (segment (start 97.427522 108.460012) (end 102.978483 108.460012) (width 0.7) (layer B.Cu) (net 25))
 (segment (start 86.36 85.09) (end 95.219993 93.949993) (width 0.7) (layer B.Cu) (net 25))
 (segment (start 104.650012 106.788483) (end 104.650012 101.157907) (width 0.7) (layer B.Cu) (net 25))
 (segment (start 115.637919 90.17) (end 116.84 90.17) (width 0.7) (layer B.Cu) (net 25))
 (segment (start 102.978483 108.460012) (end 104.650012 106.788483) (width 0.7) (layer B.Cu) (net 25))
 (segment (start 104.650012 101.157907) (end 115.637919 90.17) (width 0.7) (layer B.Cu) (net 25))
 (segment (start 93.919978 95.189978) (end 93.919978 106.790966) (width 0.7) (layer B.Cu) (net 23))
 (segment (start 115.637919 92.71) (end 116.84 92.71) (width 0.7) (layer B.Cu) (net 23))
 (segment (start 105.950023 102.397896) (end 115.637919 92.71) (width 0.7) (layer B.Cu) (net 23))
 (segment (start 93.919978 106.790966) (end 96.889035 109.760023) (width 0.7) (layer B.Cu) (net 23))
 (segment (start 96.889035 109.760023) (end 103.516965 109.760023) (width 0.7) (layer B.Cu) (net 23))
 (segment (start 103.516965 109.760023) (end 105.950023 107.326965) (width 0.7) (layer B.Cu) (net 23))
 (segment (start 86.36 87.63) (end 93.919978 95.189978) (width 0.7) (layer B.Cu) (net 23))
 (segment (start 105.950023 107.326965) (end 105.950023 102.397896) (width 0.7) (layer B.Cu) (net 23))
 (segment (start 104.055447 111.060034) (end 107.250034 107.865447) (width 0.7) (layer B.Cu) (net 21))
 (segment (start 86.36 90.17) (end 92.619967 96.429967) (width 0.7) (layer B.Cu) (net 21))
 (segment (start 92.619967 96.429967) (end 92.619967 107.329448) (width 0.7) (layer B.Cu) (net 21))
 (segment (start 115.637919 95.25) (end 116.84 95.25) (width 0.7) (layer B.Cu) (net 21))
 (segment (start 107.250034 107.865447) (end 107.250034 103.637885) (width 0.7) (layer B.Cu) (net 21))
 (segment (start 92.619967 107.329448) (end 96.350553 111.060034) (width 0.7) (layer B.Cu) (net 21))
 (segment (start 96.350553 111.060034) (end 104.055447 111.060034) (width 0.7) (layer B.Cu) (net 21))
 (segment (start 107.250034 103.637885) (end 115.637919 95.25) (width 0.7) (layer B.Cu) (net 21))
 (segment (start 108.550045 104.877874) (end 115.637919 97.79) (width 0.7) (layer B.Cu) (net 19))
 (segment (start 104.593929 112.360045) (end 108.550045 108.403929) (width 0.7) (layer B.Cu) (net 19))
 (segment (start 95.812071 112.360045) (end 104.593929 112.360045) (width 0.7) (layer B.Cu) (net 19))
 (segment (start 91.31996 107.867934) (end 95.812071 112.360045) (width 0.7) (layer B.Cu) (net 19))
 (segment (start 91.31996 97.66996) (end 91.31996 107.867934) (width 0.7) (layer B.Cu) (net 19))
 (segment (start 86.36 92.71) (end 91.31996 97.66996) (width 0.7) (layer B.Cu) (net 19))
 (segment (start 108.550045 108.403929) (end 108.550045 104.877874) (width 0.7) (layer B.Cu) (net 19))
 (segment (start 115.637919 97.79) (end 116.84 97.79) (width 0.7) (layer B.Cu) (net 19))
 (segment (start 115.637919 100.33) (end 116.84 100.33) (width 0.7) (layer B.Cu) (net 17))
 (segment (start 109.850056 106.117863) (end 115.637919 100.33) (width 0.7) (layer B.Cu) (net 17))
 (segment (start 109.850056 108.942411) (end 109.850056 106.117863) (width 0.7) (layer B.Cu) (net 17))
 (segment (start 105.132411 113.660056) (end 109.850056 108.942411) (width 0.7) (layer B.Cu) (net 17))
 (segment (start 95.273589 113.660056) (end 105.132411 113.660056) (width 0.7) (layer B.Cu) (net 17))
 (segment (start 90.555944 108.942411) (end 95.273589 113.660056) (width 0.7) (layer B.Cu) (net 17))
 (segment (start 90.555944 108.942406) (end 90.555944 108.942411) (width 0.7) (layer B.Cu) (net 17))
 (segment (start 90.019949 108.406411) (end 90.555944 108.942406) (width 0.7) (layer B.Cu) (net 17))
 (segment (start 86.36 95.25) (end 90.019949 98.909949) (width 0.7) (layer B.Cu) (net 17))
 (segment (start 90.019949 98.909949) (end 90.019949 108.406411) (width 0.7) (layer B.Cu) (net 17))
 (segment (start 87.159999 98.589999) (end 86.36 97.79) (width 0.7) (layer B.Cu) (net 16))
 (segment (start 88.719939 108.944892) (end 88.719939 100.149939) (width 0.7) (layer B.Cu) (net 16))
 (segment (start 94.735113 114.960066) (end 88.719939 108.944892) (width 0.7) (layer B.Cu) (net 16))
 (segment (start 111.150066 109.480892) (end 105.670892 114.960066) (width 0.7) (layer B.Cu) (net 16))
 (segment (start 105.670892 114.960066) (end 94.735113 114.960066) (width 0.7) (layer B.Cu) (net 16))
 (segment (start 111.150066 107.357853) (end 111.150066 109.480892) (width 0.7) (layer B.Cu) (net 16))
 (segment (start 115.637919 102.87) (end 111.150066 107.357853) (width 0.7) (layer B.Cu) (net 16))
 (segment (start 88.719939 100.149939) (end 87.159999 98.589999) (width 0.7) (layer B.Cu) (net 16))
 (segment (start 116.84 102.87) (end 115.637919 102.87) (width 0.7) (layer B.Cu) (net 16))
 (via (at 113.03 113.03) (size 1.6) (drill 0.8) (layers F.Cu B.Cu) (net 34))
 (segment (start 115.57 110.49) (end 113.03 113.03) (width 0.7) (layer B.Cu) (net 34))
 (segment (start 116.84 110.49) (end 115.57 110.49) (width 0.7) (layer B.Cu) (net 34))
 (segment (start 86.36 72.39) (end 88.9 72.39) (width 0.7) (layer B.Cu) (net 34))
 (via (at 88.9 72.39) (size 1.6) (drill 0.8) (layers F.Cu B.Cu) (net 34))
 (segment (start 67.31 73.66) (end 61.468 73.66) (width 0.7) (layer B.Cu) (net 37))
 (segment (start 61.468 73.66) (end 56.896 78.232) (width 0.7) (layer B.Cu) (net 37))
 (segment (start 58.487919 90.17) (end 59.69 90.17) (width 0.7) (layer B.Cu) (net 37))
 (segment (start 56.896 78.232) (end 56.896 88.578081) (width 0.7) (layer B.Cu) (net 37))
 (segment (start 56.896 88.578081) (end 58.487919 90.17) (width 0.7) (layer B.Cu) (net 37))
 (via (at 113.031397 107.951397) (size 1.6) (drill 0.8) (layers F.Cu B.Cu) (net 14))
 (segment (start 116.84 105.41) (end 115.572794 105.41) (width 0.7) (layer B.Cu) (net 14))
 (segment (start 115.572794 105.41) (end 113.031397 107.951397) (width 0.7) (layer B.Cu) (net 14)))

